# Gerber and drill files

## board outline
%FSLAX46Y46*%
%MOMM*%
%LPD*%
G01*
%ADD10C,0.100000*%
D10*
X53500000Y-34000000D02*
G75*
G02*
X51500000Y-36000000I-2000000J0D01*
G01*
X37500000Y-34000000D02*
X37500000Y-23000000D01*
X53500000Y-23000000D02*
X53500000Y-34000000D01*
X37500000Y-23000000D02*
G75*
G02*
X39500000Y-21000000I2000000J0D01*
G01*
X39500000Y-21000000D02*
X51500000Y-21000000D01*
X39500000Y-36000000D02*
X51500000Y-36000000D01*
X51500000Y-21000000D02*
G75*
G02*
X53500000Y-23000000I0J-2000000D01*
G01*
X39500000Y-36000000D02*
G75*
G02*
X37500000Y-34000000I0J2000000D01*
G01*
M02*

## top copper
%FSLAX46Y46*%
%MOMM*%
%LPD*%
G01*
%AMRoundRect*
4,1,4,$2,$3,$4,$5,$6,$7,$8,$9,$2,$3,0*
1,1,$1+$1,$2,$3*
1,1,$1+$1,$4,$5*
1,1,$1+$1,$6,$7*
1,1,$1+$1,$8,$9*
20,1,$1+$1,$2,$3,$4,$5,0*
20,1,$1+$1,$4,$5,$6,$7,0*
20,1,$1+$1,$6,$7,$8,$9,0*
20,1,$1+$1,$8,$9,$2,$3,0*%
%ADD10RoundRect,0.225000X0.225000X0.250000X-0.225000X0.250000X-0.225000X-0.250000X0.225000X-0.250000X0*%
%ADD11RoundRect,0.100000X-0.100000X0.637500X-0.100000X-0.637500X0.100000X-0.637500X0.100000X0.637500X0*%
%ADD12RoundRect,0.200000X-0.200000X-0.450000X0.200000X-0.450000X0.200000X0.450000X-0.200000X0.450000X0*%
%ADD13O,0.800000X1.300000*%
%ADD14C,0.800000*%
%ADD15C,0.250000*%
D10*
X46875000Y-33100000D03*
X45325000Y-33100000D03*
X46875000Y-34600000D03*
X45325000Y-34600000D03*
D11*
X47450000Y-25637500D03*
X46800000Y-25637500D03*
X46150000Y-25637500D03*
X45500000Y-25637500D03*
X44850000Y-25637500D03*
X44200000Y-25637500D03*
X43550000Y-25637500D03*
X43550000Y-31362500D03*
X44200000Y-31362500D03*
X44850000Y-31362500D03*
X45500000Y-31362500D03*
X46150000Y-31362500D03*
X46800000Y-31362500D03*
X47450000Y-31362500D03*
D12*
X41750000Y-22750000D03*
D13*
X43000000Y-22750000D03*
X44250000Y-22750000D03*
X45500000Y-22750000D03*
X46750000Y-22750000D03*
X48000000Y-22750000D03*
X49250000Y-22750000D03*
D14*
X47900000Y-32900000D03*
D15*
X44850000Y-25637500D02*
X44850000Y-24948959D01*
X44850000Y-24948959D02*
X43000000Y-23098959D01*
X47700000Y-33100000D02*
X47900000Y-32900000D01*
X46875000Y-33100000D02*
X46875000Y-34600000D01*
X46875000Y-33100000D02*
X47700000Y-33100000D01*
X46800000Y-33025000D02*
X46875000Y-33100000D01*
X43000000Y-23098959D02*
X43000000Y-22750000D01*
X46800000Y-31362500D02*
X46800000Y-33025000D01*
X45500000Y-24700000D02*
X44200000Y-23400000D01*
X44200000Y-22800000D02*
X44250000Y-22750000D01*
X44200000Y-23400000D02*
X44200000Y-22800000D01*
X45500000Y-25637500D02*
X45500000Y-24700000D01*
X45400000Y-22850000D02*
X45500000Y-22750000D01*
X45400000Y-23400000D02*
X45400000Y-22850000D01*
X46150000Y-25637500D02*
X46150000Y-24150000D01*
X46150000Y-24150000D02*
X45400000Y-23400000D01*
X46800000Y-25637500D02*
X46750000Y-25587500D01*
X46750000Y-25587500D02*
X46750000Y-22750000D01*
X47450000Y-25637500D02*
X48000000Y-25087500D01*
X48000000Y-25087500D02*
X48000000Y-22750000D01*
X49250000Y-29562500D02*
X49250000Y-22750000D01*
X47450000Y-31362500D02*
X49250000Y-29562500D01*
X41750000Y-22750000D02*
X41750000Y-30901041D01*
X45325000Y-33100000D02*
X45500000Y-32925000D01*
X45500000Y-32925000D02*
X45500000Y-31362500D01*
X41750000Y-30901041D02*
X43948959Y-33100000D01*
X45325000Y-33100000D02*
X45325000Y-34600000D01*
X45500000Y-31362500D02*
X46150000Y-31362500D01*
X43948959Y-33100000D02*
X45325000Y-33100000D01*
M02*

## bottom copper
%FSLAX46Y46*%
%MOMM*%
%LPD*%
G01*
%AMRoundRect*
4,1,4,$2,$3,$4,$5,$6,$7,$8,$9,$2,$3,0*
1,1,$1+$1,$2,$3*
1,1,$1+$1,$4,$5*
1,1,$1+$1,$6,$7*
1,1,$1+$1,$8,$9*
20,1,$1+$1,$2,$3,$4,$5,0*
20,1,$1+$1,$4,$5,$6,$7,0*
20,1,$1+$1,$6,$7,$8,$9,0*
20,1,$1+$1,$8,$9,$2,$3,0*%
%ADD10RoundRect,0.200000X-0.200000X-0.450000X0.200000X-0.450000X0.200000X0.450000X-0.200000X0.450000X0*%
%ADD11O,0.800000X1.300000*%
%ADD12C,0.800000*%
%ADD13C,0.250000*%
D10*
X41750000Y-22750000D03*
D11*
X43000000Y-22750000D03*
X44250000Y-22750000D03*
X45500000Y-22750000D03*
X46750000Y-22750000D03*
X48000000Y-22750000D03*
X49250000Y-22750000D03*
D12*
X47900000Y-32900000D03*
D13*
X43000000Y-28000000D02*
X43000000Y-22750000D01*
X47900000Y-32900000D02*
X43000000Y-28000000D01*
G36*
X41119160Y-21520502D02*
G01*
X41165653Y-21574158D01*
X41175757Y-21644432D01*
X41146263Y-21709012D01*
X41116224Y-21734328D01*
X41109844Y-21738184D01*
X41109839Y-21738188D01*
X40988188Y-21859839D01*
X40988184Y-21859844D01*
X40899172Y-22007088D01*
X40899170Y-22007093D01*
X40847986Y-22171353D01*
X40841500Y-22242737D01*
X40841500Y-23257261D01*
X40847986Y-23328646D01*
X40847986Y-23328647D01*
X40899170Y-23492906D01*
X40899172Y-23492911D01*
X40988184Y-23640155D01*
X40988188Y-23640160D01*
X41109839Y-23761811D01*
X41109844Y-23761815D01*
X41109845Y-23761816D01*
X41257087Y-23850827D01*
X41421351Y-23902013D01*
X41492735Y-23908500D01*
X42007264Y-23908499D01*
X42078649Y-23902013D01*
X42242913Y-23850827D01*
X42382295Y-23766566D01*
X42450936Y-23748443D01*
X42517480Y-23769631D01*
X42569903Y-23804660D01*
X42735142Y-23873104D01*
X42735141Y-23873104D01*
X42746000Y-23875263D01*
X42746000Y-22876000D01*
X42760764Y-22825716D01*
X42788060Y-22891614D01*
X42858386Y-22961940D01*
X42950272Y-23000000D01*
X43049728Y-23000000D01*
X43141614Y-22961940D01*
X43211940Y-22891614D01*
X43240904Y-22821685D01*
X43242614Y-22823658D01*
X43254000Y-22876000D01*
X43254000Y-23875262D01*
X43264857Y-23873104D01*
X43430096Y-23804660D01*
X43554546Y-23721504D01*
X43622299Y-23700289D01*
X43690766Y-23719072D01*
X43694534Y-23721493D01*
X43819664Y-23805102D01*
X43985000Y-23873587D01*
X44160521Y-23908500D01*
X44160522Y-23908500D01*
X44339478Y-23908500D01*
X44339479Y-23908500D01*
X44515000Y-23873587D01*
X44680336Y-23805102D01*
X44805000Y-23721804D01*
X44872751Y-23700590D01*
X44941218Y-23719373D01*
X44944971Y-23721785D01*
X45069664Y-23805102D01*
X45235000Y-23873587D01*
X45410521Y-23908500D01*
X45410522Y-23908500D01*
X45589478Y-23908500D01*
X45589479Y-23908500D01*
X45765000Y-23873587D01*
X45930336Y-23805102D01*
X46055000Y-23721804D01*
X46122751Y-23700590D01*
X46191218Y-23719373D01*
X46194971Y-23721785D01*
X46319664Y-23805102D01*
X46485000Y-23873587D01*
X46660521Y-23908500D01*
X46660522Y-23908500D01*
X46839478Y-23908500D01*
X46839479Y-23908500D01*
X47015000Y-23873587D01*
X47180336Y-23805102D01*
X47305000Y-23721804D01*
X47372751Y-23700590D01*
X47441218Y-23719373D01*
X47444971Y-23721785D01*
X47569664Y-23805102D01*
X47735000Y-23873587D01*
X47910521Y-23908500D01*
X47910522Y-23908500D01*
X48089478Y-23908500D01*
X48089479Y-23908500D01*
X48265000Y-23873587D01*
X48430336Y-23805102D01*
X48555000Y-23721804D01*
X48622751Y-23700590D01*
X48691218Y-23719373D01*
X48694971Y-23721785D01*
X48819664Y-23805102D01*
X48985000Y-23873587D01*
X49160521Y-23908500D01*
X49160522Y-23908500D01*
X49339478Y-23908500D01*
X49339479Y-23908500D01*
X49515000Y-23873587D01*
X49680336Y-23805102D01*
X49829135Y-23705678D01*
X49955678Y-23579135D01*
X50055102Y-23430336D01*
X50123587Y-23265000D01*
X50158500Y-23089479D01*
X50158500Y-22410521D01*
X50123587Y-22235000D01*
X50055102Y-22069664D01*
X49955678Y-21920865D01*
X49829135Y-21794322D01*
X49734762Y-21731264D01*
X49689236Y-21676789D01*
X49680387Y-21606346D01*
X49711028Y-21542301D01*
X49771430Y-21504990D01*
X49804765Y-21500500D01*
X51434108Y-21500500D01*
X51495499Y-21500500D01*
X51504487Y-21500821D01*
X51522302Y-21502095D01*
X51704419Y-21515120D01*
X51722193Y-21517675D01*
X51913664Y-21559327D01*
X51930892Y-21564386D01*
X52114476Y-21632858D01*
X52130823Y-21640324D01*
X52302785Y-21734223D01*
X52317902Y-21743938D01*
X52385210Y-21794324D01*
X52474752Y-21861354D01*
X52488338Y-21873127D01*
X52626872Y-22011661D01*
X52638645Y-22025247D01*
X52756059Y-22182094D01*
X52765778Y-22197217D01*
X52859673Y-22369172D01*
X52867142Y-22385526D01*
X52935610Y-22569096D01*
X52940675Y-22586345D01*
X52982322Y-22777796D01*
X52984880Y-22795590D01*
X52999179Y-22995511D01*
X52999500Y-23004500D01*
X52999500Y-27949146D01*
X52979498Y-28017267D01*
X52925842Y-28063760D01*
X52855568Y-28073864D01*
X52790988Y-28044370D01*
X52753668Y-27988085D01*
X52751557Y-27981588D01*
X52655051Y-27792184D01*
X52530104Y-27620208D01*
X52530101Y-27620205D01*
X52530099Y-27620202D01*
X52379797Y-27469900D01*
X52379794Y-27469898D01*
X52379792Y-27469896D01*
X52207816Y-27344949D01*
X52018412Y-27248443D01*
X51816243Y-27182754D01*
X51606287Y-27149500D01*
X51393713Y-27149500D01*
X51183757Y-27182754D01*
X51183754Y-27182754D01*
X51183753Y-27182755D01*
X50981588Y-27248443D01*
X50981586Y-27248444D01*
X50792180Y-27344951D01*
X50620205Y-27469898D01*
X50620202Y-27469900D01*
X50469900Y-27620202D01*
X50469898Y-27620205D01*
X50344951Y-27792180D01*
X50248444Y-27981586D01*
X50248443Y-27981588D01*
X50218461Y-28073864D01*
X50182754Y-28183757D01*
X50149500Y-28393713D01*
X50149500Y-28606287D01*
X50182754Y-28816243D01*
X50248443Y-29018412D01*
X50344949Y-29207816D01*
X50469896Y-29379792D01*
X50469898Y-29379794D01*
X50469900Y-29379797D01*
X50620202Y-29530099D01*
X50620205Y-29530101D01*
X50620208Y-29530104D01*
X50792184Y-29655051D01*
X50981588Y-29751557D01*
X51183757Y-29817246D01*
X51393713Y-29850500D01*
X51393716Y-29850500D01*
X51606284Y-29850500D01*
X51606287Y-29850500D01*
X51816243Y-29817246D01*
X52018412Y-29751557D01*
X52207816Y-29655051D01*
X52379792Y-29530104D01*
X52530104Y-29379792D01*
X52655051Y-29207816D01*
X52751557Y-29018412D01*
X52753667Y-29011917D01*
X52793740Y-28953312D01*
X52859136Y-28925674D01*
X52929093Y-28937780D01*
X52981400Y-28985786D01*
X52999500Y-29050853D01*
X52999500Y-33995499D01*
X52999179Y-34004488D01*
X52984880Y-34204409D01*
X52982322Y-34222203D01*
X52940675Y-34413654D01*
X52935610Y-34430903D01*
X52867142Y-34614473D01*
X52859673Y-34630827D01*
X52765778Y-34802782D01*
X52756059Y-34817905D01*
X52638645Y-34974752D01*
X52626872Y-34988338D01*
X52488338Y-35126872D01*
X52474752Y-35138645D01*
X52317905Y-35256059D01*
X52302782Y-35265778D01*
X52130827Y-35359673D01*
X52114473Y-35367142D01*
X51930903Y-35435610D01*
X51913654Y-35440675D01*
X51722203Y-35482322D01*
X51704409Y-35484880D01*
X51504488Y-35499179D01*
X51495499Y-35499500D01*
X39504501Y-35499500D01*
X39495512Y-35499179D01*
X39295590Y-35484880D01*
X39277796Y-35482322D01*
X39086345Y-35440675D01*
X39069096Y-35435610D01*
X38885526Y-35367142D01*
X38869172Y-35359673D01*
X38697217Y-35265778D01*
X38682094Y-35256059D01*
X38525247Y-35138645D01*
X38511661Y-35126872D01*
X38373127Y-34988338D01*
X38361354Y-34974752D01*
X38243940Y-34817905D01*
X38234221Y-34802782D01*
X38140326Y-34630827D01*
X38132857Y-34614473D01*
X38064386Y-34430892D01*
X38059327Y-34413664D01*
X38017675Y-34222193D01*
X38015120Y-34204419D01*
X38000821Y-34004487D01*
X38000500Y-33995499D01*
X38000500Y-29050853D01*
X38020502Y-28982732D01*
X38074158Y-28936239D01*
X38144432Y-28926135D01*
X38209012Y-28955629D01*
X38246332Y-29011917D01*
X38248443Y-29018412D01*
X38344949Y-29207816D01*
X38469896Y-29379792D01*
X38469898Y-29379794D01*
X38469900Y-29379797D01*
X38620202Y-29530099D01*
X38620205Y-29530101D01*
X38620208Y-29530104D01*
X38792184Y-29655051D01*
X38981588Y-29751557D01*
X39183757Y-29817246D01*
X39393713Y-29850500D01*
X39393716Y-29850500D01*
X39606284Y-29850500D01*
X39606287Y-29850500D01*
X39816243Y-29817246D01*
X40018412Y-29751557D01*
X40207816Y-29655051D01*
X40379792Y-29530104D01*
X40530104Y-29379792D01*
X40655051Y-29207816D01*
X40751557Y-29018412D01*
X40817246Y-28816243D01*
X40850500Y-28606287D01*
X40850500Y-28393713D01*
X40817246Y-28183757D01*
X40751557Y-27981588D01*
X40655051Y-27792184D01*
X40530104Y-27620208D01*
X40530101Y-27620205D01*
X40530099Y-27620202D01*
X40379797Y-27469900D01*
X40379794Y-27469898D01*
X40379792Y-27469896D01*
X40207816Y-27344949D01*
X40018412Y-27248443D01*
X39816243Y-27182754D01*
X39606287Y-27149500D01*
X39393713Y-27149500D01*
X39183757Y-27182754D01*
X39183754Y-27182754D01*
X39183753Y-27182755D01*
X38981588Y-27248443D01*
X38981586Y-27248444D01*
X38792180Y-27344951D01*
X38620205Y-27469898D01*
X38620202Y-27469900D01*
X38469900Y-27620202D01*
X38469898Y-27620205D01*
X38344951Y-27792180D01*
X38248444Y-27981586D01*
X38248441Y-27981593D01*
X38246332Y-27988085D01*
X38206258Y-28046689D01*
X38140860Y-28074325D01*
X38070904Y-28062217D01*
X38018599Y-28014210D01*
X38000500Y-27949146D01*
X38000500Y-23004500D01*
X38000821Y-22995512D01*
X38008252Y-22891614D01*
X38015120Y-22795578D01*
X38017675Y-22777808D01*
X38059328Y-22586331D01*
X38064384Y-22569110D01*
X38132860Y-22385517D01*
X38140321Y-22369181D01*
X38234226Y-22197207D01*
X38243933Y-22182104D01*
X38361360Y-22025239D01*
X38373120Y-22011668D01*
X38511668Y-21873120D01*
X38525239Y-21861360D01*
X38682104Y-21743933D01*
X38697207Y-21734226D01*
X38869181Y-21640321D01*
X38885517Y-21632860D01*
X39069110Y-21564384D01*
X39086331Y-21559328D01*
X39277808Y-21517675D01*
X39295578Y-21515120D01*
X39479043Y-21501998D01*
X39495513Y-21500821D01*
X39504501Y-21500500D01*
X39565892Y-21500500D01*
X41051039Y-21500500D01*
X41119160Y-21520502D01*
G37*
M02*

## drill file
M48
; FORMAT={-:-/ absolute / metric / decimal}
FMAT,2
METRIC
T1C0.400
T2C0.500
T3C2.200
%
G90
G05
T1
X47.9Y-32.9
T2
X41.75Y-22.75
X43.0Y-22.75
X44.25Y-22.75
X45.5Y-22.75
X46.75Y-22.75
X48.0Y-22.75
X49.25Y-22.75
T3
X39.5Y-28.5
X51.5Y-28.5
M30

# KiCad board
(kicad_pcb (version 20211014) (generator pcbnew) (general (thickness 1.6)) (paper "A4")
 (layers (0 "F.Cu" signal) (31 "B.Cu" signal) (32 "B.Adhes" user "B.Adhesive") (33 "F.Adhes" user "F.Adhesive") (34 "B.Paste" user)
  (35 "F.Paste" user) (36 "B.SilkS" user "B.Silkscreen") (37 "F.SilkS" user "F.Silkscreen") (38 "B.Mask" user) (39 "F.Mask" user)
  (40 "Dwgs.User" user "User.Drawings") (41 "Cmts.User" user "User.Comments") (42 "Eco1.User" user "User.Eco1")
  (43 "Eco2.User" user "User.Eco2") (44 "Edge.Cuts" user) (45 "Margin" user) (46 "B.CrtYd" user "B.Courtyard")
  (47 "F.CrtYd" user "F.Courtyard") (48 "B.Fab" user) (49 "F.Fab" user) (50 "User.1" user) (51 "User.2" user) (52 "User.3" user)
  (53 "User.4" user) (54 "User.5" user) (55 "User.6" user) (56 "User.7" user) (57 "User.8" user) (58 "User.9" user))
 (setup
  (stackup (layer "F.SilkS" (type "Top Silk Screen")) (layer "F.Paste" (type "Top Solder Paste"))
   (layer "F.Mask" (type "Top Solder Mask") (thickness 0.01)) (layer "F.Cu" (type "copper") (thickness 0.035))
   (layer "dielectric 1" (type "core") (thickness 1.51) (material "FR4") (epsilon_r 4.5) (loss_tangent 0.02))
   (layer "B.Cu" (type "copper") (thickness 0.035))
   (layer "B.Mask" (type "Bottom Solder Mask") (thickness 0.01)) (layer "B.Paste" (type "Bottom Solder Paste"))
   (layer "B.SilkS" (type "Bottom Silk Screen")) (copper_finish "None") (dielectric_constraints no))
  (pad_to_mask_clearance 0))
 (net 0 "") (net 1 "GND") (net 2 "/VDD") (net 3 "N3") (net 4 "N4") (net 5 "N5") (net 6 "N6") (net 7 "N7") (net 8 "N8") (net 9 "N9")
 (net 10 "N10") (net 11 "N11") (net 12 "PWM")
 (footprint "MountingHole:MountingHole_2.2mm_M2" (layer "F.Cu") (at 39.5 28.5)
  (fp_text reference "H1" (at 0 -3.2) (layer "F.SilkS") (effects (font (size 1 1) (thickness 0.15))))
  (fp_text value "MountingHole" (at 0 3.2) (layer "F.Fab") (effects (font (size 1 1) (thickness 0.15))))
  (pad "" np_thru_hole circle (at 0 0) (size 2.2 2.2) (drill 2.2) (layers *.Cu *.Mask)))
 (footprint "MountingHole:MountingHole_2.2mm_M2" (layer "F.Cu") (at 51.5 28.5)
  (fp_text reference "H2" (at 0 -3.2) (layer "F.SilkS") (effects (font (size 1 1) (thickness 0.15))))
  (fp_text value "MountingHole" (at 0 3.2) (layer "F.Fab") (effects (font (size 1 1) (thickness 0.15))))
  (pad "" np_thru_hole circle (at 0 0) (size 2.2 2.2) (drill 2.2) (layers *.Cu *.Mask)))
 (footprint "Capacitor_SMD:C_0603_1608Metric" (layer "F.Cu") (at 46.1 33.1 180)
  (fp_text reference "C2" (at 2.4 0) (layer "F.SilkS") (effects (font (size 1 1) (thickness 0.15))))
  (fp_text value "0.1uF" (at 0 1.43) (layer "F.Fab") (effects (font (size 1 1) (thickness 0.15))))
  (pad "1" smd roundrect (at -0.775 0 180) (size 0.9 0.95) (layers "F.Cu" "F.Paste" "F.Mask") (roundrect_rratio 0.25) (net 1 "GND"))
  (pad "2" smd roundrect (at 0.775 0 180) (size 0.9 0.95) (layers "F.Cu" "F.Paste" "F.Mask") (roundrect_rratio 0.25) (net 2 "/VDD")))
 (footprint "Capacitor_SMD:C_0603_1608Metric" (layer "F.Cu") (at 46.1 34.6 180)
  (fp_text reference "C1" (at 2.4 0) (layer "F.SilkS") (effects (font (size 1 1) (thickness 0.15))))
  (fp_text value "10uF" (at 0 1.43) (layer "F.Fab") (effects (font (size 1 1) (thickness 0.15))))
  (pad "1" smd roundrect (at -0.775 0 180) (size 0.9 0.95) (layers "F.Cu" "F.Paste" "F.Mask") (roundrect_rratio 0.25) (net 1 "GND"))
  (pad "2" smd roundrect (at 0.775 0 180) (size 0.9 0.95) (layers "F.Cu" "F.Paste" "F.Mask") (roundrect_rratio 0.25) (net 2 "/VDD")))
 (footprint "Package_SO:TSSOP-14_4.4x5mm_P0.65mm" (layer "F.Cu") (at 45.5 28.5 -90)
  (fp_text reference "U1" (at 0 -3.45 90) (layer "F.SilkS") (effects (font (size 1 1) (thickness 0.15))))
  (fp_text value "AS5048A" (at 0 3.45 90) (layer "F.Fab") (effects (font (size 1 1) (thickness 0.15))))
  (pad "1" smd roundrect (at -2.8625 -1.95 270) (size 1.475 0.4) (layers "F.Cu" "F.Paste" "F.Mask") (roundrect_rratio 0.25) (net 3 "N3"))
  (pad "2" smd roundrect (at -2.8625 -1.3 270) (size 1.475 0.4) (layers "F.Cu" "F.Paste" "F.Mask") (roundrect_rratio 0.25) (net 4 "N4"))
  (pad "3" smd roundrect (at -2.8625 -0.65 270) (size 1.475 0.4) (layers "F.Cu" "F.Paste" "F.Mask") (roundrect_rratio 0.25) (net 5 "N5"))
  (pad "4" smd roundrect (at -2.8625 0 270) (size 1.475 0.4) (layers "F.Cu" "F.Paste" "F.Mask") (roundrect_rratio 0.25) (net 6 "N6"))
  (pad "5" smd roundrect (at -2.8625 0.65 270) (size 1.475 0.4) (layers "F.Cu" "F.Paste" "F.Mask") (roundrect_rratio 0.25) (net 1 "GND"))
  (pad "6" smd roundrect (at -2.8625 1.3 270) (size 1.475 0.4) (layers "F.Cu" "F.Paste" "F.Mask") (roundrect_rratio 0.25) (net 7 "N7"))
  (pad "7" smd roundrect (at -2.8625 1.95 270) (size 1.475 0.4) (layers "F.Cu" "F.Paste" "F.Mask") (roundrect_rratio 0.25) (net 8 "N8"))
  (pad "8" smd roundrect (at 2.8625 1.95 270) (size 1.475 0.4) (layers "F.Cu" "F.Paste" "F.Mask") (roundrect_rratio 0.25) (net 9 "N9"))
  (pad "9" smd roundrect (at 2.8625 1.3 270) (size 1.475 0.4) (layers "F.Cu" "F.Paste" "F.Mask") (roundrect_rratio 0.25) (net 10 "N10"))
  (pad "10" smd roundrect (at 2.8625 0.65 270) (size 1.475 0.4) (layers "F.Cu" "F.Paste" "F.Mask") (roundrect_rratio 0.25) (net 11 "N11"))
  (pad "11" smd roundrect (at 2.8625 0 270) (size 1.475 0.4) (layers "F.Cu" "F.Paste" "F.Mask") (roundrect_rratio 0.25) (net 2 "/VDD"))
  (pad "12" smd roundrect (at 2.8625 -0.65 270) (size 1.475 0.4) (layers "F.Cu" "F.Paste" "F.Mask") (roundrect_rratio 0.25) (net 2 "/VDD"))
  (pad "13" smd roundrect (at 2.8625 -1.3 270) (size 1.475 0.4) (layers "F.Cu" "F.Paste" "F.Mask") (roundrect_rratio 0.25) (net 1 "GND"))
  (pad "14" smd roundrect (at 2.8625 -1.95 270) (size 1.475 0.4) (layers "F.Cu" "F.Paste" "F.Mask") (roundrect_rratio 0.25) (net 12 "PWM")))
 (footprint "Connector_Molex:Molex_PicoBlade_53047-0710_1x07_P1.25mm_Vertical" (layer "B.Cu") (at 41.75 22.75)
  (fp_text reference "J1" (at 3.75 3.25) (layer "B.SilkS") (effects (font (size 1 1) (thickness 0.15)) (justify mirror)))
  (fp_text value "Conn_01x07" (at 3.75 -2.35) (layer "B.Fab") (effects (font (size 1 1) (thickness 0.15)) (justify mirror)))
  (pad "1" thru_hole roundrect (at 0 0) (size 0.8 1.3) (drill 0.5) (layers *.Cu *.Mask) (roundrect_rratio 0.25) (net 2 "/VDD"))
  (pad "2" thru_hole oval (at 1.25 0) (size 0.8 1.3) (drill 0.5) (layers *.Cu *.Mask) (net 1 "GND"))
  (pad "3" thru_hole oval (at 2.5 0) (size 0.8 1.3) (drill 0.5) (layers *.Cu *.Mask) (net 6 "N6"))
  (pad "4" thru_hole oval (at 3.75 0) (size 0.8 1.3) (drill 0.5) (layers *.Cu *.Mask) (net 5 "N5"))
  (pad "5" thru_hole oval (at 5 0) (size 0.8 1.3) (drill 0.5) (layers *.Cu *.Mask) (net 4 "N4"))
  (pad "6" thru_hole oval (at 6.25 0) (size 0.8 1.3) (drill 0.5) (layers *.Cu *.Mask) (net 3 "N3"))
  (pad "7" thru_hole oval (at 7.5 0) (size 0.8 1.3) (drill 0.5) (layers *.Cu *.Mask) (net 12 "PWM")))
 (gr_arc (start 53.5 34) (mid 52.914214 35.414214) (end 51.5 36) (layer "Edge.Cuts") (width 0.1))
 (gr_line (start 37.5 34) (end 37.5 23) (layer "Edge.Cuts") (width 0.1))
 (gr_line (start 53.5 23) (end 53.5 34) (layer "Edge.Cuts") (width 0.1))
 (gr_arc (start 37.5 23) (mid 38.085786 21.585786) (end 39.5 21) (layer "Edge.Cuts") (width 0.1))
 (gr_line (start 39.5 21) (end 51.5 21) (layer "Edge.Cuts") (width 0.1))
 (gr_line (start 39.5 36) (end 51.5 36) (layer "Edge.Cuts") (width 0.1))
 (gr_arc (start 51.5 21) (mid 52.914214 21.585786) (end 53.5 23) (layer "Edge.Cuts") (width 0.1))
 (gr_arc (start 39.5 36) (mid 38.085786 35.414214) (end 37.5 34) (layer "Edge.Cuts") (width 0.1))
 (segment (start 44.85 25.6375) (end 44.85 24.948959) (width 0.25) (layer "F.Cu") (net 1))
 (segment (start 44.85 24.948959) (end 43 23.098959) (width 0.25) (layer "F.Cu") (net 1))
 (segment (start 47.7 33.1) (end 47.9 32.9) (width 0.25) (layer "F.Cu") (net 1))
 (segment (start 46.875 33.1) (end 46.875 34.6) (width 0.25) (layer "F.Cu") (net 1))
 (segment (start 46.875 33.1) (end 47.7 33.1) (width 0.25) (layer "F.Cu") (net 1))
 (segment (start 46.8 33.025) (end 46.875 33.1) (width 0.25) (layer "F.Cu") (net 1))
 (segment (start 43 23.098959) (end 43 22.75) (width 0.25) (layer "F.Cu") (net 1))
 (segment (start 46.8 31.3625) (end 46.8 33.025) (width 0.25) (layer "F.Cu") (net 1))
 (via (at 47.9 32.9) (size 0.8) (drill 0.4) (layers "F.Cu" "B.Cu") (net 1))
 (segment (start 43 28) (end 43 22.75) (width 0.25) (layer "B.Cu") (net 1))
 (segment (start 47.9 32.9) (end 43 28) (width 0.25) (layer "B.Cu") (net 1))
 (segment (start 45.5 24.7) (end 44.2 23.4) (width 0.25) (layer "F.Cu") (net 6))
 (segment (start 44.2 22.8) (end 44.25 22.75) (width 0.25) (layer "F.Cu") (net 6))
 (segment (start 44.2 23.4) (end 44.2 22.8) (width 0.25) (layer "F.Cu") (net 6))
 (segment (start 45.5 25.6375) (end 45.5 24.7) (width 0.25) (layer "F.Cu") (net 6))
 (segment (start 45.4 22.85) (end 45.5 22.75) (width 0.25) (layer "F.Cu") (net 5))
 (segment (start 45.4 23.4) (end 45.4 22.85) (width 0.25) (layer "F.Cu") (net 5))
 (segment (start 46.15 25.6375) (end 46.15 24.15) (width 0.25) (layer "F.Cu") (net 5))
 (segment (start 46.15 24.15) (end 45.4 23.4) (width 0.25) (layer "F.Cu") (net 5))
 (segment (start 46.8 25.6375) (end 46.75 25.5875) (width 0.25) (layer "F.Cu") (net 4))
 (segment (start 46.75 25.5875) (end 46.75 22.75) (width 0.25) (layer "F.Cu") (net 4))
 (segment (start 47.45 25.6375) (end 48 25.0875) (width 0.25) (layer "F.Cu") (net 3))
 (segment (start 48 25.0875) (end 48 22.75) (width 0.25) (layer "F.Cu") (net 3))
 (segment (start 49.25 29.5625) (end 49.25 22.75) (width 0.25) (layer "F.Cu") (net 12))
 (segment (start 47.45 31.3625) (end 49.25 29.5625) (width 0.25) (layer "F.Cu") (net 12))
 (segment (start 41.75 22.75) (end 41.75 30.901041) (width 0.25) (layer "F.Cu") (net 2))
 (segment (start 45.325 33.1) (end 45.5 32.925) (width 0.25) (layer "F.Cu") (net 2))
 (segment (start 45.5 32.925) (end 45.5 31.3625) (width 0.25) (layer "F.Cu") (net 2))
 (segment (start 41.75 30.901041) (end 43.948959 33.1) (width 0.25) (layer "F.Cu") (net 2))
 (segment (start 45.325 33.1) (end 45.325 34.6) (width 0.25) (layer "F.Cu") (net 2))
 (segment (start 45.5 31.3625) (end 46.15 31.3625) (width 0.25) (layer "F.Cu") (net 2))
 (segment (start 43.948959 33.1) (end 45.325 33.1) (width 0.25) (layer "F.Cu") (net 2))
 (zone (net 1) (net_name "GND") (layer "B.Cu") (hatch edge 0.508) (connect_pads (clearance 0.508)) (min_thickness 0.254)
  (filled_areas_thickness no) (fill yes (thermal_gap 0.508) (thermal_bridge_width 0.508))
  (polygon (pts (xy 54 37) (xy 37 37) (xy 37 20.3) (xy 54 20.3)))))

